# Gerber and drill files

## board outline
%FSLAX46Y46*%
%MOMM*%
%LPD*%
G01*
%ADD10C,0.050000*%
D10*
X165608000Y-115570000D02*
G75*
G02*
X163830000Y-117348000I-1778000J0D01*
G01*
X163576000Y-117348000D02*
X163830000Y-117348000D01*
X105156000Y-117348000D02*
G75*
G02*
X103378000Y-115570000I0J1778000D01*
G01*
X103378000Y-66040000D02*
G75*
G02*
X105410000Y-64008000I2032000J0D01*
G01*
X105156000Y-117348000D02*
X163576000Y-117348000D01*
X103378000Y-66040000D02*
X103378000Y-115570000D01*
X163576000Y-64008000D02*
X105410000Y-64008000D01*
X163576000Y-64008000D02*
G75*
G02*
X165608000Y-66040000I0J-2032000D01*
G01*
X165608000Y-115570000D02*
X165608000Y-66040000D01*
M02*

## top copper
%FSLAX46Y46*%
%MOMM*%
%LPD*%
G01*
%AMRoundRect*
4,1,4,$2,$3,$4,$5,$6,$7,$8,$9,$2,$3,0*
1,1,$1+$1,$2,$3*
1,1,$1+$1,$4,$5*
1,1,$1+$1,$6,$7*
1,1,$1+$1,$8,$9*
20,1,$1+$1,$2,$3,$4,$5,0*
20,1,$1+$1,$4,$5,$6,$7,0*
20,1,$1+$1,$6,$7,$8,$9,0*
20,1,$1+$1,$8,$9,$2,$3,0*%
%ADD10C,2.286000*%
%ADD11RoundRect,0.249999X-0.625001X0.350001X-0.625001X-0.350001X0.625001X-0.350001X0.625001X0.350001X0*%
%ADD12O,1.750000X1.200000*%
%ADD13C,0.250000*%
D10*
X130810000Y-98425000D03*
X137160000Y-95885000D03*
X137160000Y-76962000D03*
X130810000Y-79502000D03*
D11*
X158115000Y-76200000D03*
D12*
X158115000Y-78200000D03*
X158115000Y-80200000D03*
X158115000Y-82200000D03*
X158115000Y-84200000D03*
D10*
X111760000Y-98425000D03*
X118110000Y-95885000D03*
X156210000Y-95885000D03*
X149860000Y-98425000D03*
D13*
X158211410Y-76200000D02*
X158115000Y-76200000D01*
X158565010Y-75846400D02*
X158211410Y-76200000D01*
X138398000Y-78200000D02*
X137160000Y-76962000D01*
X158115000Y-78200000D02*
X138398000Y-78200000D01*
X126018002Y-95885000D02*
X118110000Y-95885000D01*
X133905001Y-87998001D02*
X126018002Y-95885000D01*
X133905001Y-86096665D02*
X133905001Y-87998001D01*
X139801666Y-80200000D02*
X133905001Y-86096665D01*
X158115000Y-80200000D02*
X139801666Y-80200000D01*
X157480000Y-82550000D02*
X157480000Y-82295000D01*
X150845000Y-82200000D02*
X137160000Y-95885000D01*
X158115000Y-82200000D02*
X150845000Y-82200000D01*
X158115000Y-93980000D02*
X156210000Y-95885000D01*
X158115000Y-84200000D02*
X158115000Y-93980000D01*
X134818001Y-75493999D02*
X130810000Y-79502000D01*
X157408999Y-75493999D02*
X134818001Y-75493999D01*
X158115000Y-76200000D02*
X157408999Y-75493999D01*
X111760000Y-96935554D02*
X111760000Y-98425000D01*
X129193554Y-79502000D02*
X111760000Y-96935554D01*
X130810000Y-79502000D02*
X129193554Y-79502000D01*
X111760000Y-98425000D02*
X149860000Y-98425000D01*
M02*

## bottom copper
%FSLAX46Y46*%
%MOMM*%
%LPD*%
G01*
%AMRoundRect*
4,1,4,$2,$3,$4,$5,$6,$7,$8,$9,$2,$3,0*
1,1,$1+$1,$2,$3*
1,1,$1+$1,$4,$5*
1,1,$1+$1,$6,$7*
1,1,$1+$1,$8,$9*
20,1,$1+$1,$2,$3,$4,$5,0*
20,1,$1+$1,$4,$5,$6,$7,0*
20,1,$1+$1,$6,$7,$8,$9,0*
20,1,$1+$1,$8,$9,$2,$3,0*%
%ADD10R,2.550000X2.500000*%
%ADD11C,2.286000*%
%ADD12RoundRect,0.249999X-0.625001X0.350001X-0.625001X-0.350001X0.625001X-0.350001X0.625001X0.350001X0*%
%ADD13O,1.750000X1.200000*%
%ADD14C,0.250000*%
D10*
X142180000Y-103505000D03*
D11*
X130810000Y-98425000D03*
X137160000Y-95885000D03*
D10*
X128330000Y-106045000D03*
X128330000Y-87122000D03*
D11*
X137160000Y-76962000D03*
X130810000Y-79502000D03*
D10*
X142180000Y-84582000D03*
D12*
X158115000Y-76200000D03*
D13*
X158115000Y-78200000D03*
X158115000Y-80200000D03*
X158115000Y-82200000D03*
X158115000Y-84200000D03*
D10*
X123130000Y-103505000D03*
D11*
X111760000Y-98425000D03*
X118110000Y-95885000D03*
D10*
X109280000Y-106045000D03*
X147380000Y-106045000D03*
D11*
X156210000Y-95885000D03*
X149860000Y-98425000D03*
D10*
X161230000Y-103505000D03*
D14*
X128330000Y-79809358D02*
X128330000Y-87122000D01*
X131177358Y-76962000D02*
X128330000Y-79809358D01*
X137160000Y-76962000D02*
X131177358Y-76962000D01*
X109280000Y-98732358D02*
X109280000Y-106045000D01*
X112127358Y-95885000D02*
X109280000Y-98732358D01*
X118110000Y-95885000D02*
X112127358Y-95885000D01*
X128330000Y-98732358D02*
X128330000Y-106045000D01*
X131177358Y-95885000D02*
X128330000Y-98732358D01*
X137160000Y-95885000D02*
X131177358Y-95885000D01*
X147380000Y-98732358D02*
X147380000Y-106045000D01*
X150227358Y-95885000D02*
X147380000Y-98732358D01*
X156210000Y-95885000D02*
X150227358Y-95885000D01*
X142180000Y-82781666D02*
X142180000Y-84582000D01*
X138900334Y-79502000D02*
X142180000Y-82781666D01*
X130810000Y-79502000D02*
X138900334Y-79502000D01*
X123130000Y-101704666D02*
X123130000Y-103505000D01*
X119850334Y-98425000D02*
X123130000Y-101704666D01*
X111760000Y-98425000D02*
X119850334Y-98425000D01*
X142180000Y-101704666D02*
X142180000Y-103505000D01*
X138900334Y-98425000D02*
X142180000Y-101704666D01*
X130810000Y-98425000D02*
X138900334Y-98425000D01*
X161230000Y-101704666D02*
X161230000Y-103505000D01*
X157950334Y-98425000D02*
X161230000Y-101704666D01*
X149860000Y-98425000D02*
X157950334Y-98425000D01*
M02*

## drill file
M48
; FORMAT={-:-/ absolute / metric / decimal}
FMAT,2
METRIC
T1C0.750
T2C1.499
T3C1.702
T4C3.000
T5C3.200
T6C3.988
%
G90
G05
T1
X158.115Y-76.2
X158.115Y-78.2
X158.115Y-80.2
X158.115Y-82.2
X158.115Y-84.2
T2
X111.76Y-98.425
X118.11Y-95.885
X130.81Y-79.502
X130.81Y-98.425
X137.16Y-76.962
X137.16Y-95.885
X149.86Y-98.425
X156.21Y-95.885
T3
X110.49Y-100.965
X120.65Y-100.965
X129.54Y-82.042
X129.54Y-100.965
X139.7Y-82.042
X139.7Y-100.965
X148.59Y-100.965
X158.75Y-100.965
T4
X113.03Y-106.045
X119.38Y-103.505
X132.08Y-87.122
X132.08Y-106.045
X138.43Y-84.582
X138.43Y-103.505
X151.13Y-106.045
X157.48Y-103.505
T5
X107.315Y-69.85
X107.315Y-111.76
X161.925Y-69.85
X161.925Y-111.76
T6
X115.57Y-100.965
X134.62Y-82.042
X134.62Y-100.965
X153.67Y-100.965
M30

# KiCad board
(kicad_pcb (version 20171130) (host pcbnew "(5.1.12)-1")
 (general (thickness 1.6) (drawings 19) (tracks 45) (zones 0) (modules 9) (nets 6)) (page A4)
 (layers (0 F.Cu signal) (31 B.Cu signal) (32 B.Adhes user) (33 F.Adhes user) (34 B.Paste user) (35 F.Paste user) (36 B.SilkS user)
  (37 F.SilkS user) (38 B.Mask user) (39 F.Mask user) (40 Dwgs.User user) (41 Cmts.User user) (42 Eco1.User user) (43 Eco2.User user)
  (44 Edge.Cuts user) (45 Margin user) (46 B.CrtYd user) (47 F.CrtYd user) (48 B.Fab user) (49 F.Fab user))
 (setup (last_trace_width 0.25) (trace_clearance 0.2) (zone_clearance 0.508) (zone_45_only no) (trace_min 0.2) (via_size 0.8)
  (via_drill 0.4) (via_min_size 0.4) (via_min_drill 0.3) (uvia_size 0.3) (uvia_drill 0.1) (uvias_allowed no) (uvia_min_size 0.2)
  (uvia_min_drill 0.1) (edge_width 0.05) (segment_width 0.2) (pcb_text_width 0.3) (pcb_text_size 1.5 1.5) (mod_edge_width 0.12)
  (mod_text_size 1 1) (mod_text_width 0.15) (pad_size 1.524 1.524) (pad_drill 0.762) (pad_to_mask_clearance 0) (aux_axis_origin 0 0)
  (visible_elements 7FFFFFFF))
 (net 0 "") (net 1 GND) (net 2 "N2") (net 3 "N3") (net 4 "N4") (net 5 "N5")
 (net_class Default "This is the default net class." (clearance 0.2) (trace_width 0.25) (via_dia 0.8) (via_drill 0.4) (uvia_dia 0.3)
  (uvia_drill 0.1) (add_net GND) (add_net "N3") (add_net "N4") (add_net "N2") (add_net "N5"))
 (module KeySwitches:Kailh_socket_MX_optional (layer F.Cu) (at 134.62 100.965)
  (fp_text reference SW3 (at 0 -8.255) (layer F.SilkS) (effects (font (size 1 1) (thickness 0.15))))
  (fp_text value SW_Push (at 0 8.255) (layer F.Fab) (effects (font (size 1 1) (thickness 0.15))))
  (pad 2 smd rect (at 7.56 2.54) (size 2.55 2.5) (layers B.Cu B.Paste B.Mask) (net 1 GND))
  (pad "" np_thru_hole circle (at -5.08 0) (size 1.7018 1.7018) (drill 1.7018) (layers *.Cu *.Mask))
  (pad "" np_thru_hole circle (at 5.08 0) (size 1.7018 1.7018) (drill 1.7018) (layers *.Cu *.Mask))
  (pad 2 thru_hole circle (at -3.81 -2.54) (size 2.286 2.286) (drill 1.4986) (layers *.Cu *.Mask) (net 1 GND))
  (pad "" np_thru_hole circle (at 0 0) (size 3.9878 3.9878) (drill 3.9878) (layers *.Cu *.Mask))
  (pad 1 thru_hole circle (at 2.54 -5.08) (size 2.286 2.286) (drill 1.4986) (layers *.Cu *.Mask) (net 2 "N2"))
  (pad "" np_thru_hole circle (at 3.81 2.54) (size 3 3) (drill 3) (layers *.Cu *.Mask))
  (pad "" np_thru_hole circle (at -2.54 5.08) (size 3 3) (drill 3) (layers *.Cu *.Mask))
  (pad 1 smd rect (at -6.29 5.08) (size 2.55 2.5) (layers B.Cu B.Paste B.Mask) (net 2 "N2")))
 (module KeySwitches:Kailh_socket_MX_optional (layer F.Cu) (at 134.62 82.042)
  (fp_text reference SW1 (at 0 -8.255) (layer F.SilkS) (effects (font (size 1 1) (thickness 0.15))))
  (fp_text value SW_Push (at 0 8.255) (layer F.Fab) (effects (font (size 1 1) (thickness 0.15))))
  (pad 1 smd rect (at -6.29 5.08) (size 2.55 2.5) (layers B.Cu B.Paste B.Mask) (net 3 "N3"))
  (pad "" np_thru_hole circle (at -2.54 5.08) (size 3 3) (drill 3) (layers *.Cu *.Mask))
  (pad "" np_thru_hole circle (at 3.81 2.54) (size 3 3) (drill 3) (layers *.Cu *.Mask))
  (pad 1 thru_hole circle (at 2.54 -5.08) (size 2.286 2.286) (drill 1.4986) (layers *.Cu *.Mask) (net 3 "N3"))
  (pad "" np_thru_hole circle (at 0 0) (size 3.9878 3.9878) (drill 3.9878) (layers *.Cu *.Mask))
  (pad 2 thru_hole circle (at -3.81 -2.54) (size 2.286 2.286) (drill 1.4986) (layers *.Cu *.Mask) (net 1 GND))
  (pad "" np_thru_hole circle (at 5.08 0) (size 1.7018 1.7018) (drill 1.7018) (layers *.Cu *.Mask))
  (pad "" np_thru_hole circle (at -5.08 0) (size 1.7018 1.7018) (drill 1.7018) (layers *.Cu *.Mask))
  (pad 2 smd rect (at 7.56 2.54) (size 2.55 2.5) (layers B.Cu B.Paste B.Mask) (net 1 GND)))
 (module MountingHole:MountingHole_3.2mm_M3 (layer F.Cu) (at 107.315 69.85)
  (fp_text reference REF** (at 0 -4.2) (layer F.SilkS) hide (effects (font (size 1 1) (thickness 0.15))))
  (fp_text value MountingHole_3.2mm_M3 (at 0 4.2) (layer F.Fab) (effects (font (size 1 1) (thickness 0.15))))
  (pad 1 np_thru_hole circle (at 0 0) (size 3.2 3.2) (drill 3.2) (layers *.Cu *.Mask)))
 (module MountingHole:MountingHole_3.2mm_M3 (layer F.Cu) (at 161.925 111.76)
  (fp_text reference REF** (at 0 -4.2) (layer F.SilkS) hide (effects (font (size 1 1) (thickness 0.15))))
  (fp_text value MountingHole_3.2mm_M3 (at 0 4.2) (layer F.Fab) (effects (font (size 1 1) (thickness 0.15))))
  (pad 1 np_thru_hole circle (at 0 0) (size 3.2 3.2) (drill 3.2) (layers *.Cu *.Mask)))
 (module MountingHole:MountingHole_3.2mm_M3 (layer F.Cu) (at 161.925 69.85)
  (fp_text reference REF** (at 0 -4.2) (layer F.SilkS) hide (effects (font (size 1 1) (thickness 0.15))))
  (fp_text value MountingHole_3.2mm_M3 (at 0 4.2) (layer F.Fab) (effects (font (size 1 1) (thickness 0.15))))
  (pad 1 np_thru_hole circle (at 0 0) (size 3.2 3.2) (drill 3.2) (layers *.Cu *.Mask)))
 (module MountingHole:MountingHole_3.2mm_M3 (layer F.Cu) (at 107.315 111.76)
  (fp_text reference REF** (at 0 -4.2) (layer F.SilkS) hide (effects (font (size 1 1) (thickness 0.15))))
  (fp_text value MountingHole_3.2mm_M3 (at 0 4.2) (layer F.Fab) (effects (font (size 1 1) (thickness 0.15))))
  (pad 1 np_thru_hole circle (at 0 0) (size 3.2 3.2) (drill 3.2) (layers *.Cu *.Mask)))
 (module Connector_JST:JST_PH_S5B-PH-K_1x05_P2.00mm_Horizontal (layer B.Cu) (at 158.115 76.2 270)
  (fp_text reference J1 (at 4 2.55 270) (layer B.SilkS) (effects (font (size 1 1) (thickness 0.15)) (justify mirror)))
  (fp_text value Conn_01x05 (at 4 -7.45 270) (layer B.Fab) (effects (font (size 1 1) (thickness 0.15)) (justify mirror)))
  (pad 1 thru_hole roundrect (at 0 0 270) (size 1.2 1.75) (drill 0.75) (layers *.Cu *.Mask) (roundrect_rratio 0.2083325) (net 1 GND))
  (pad 2 thru_hole oval (at 2 0 270) (size 1.2 1.75) (drill 0.75) (layers *.Cu *.Mask) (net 3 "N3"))
  (pad 3 thru_hole oval (at 4 0 270) (size 1.2 1.75) (drill 0.75) (layers *.Cu *.Mask) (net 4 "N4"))
  (pad 4 thru_hole oval (at 6 0 270) (size 1.2 1.75) (drill 0.75) (layers *.Cu *.Mask) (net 2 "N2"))
  (pad 5 thru_hole oval (at 8 0 270) (size 1.2 1.75) (drill 0.75) (layers *.Cu *.Mask) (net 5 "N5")))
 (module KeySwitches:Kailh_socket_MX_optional (layer F.Cu) (at 115.57 100.965)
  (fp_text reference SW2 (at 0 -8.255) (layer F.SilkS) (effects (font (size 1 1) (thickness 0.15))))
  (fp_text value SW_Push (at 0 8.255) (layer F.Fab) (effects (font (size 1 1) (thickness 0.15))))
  (pad 2 smd rect (at 7.56 2.54) (size 2.55 2.5) (layers B.Cu B.Paste B.Mask) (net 1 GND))
  (pad "" np_thru_hole circle (at -5.08 0) (size 1.7018 1.7018) (drill 1.7018) (layers *.Cu *.Mask))
  (pad "" np_thru_hole circle (at 5.08 0) (size 1.7018 1.7018) (drill 1.7018) (layers *.Cu *.Mask))
  (pad 2 thru_hole circle (at -3.81 -2.54) (size 2.286 2.286) (drill 1.4986) (layers *.Cu *.Mask) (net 1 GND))
  (pad "" np_thru_hole circle (at 0 0) (size 3.9878 3.9878) (drill 3.9878) (layers *.Cu *.Mask))
  (pad 1 thru_hole circle (at 2.54 -5.08) (size 2.286 2.286) (drill 1.4986) (layers *.Cu *.Mask) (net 4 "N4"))
  (pad "" np_thru_hole circle (at 3.81 2.54) (size 3 3) (drill 3) (layers *.Cu *.Mask))
  (pad "" np_thru_hole circle (at -2.54 5.08) (size 3 3) (drill 3) (layers *.Cu *.Mask))
  (pad 1 smd rect (at -6.29 5.08) (size 2.55 2.5) (layers B.Cu B.Paste B.Mask) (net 4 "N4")))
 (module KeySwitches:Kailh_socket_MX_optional (layer F.Cu) (at 153.67 100.965)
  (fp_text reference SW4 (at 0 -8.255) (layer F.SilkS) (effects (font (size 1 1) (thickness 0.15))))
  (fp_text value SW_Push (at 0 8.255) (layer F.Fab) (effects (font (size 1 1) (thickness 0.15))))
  (pad 1 smd rect (at -6.29 5.08) (size 2.55 2.5) (layers B.Cu B.Paste B.Mask) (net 5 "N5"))
  (pad "" np_thru_hole circle (at -2.54 5.08) (size 3 3) (drill 3) (layers *.Cu *.Mask))
  (pad "" np_thru_hole circle (at 3.81 2.54) (size 3 3) (drill 3) (layers *.Cu *.Mask))
  (pad 1 thru_hole circle (at 2.54 -5.08) (size 2.286 2.286) (drill 1.4986) (layers *.Cu *.Mask) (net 5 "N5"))
  (pad "" np_thru_hole circle (at 0 0) (size 3.9878 3.9878) (drill 3.9878) (layers *.Cu *.Mask))
  (pad 2 thru_hole circle (at -3.81 -2.54) (size 2.286 2.286) (drill 1.4986) (layers *.Cu *.Mask) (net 1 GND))
  (pad "" np_thru_hole circle (at 5.08 0) (size 1.7018 1.7018) (drill 1.7018) (layers *.Cu *.Mask))
  (pad "" np_thru_hole circle (at -5.08 0) (size 1.7018 1.7018) (drill 1.7018) (layers *.Cu *.Mask))
  (pad 2 smd rect (at 7.56 2.54) (size 2.55 2.5) (layers B.Cu B.Paste B.Mask) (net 1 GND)))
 (gr_arc (start 163.83 115.57) (end 163.83 117.348) (angle -90) (layer Edge.Cuts) (width 0.05))
 (gr_line (start 163.576 117.348) (end 163.83 117.348) (layer Edge.Cuts) (width 0.05))
 (gr_arc (start 105.156 115.57) (end 103.378 115.57) (angle -90) (layer Edge.Cuts) (width 0.05))
 (gr_arc (start 105.41 66.04) (end 105.41 64.008) (angle -90) (layer Edge.Cuts) (width 0.05))
 (gr_line (start 105.156 117.348) (end 163.576 117.348) (layer Edge.Cuts) (width 0.05))
 (gr_line (start 103.378 66.04) (end 103.378 115.57) (layer Edge.Cuts) (width 0.05))
 (gr_line (start 163.576 64.008) (end 105.41 64.008) (layer Edge.Cuts) (width 0.05))
 (gr_arc (start 163.576 66.04) (end 165.608 66.04) (angle -90) (layer Edge.Cuts) (width 0.05))
 (gr_line (start 165.608 115.57) (end 165.608 66.04) (layer Edge.Cuts) (width 0.05))
 (segment (start 158.21141 76.2) (end 158.115 76.2) (width 0.25) (layer F.Cu) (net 1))
 (segment (start 158.56501 75.8464) (end 158.21141 76.2) (width 0.25) (layer F.Cu) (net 1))
 (segment (start 138.398 78.2) (end 137.16 76.962) (width 0.25) (layer F.Cu) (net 3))
 (segment (start 158.115 78.2) (end 138.398 78.2) (width 0.25) (layer F.Cu) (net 3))
 (segment (start 128.33 79.809358) (end 128.33 87.122) (width 0.25) (layer B.Cu) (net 3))
 (segment (start 131.177358 76.962) (end 128.33 79.809358) (width 0.25) (layer B.Cu) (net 3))
 (segment (start 137.16 76.962) (end 131.177358 76.962) (width 0.25) (layer B.Cu) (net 3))
 (segment (start 126.018002 95.885) (end 118.11 95.885) (width 0.25) (layer F.Cu) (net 4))
 (segment (start 133.905001 87.998001) (end 126.018002 95.885) (width 0.25) (layer F.Cu) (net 4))
 (segment (start 133.905001 86.096665) (end 133.905001 87.998001) (width 0.25) (layer F.Cu) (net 4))
 (segment (start 139.801666 80.2) (end 133.905001 86.096665) (width 0.25) (layer F.Cu) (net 4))
 (segment (start 158.115 80.2) (end 139.801666 80.2) (width 0.25) (layer F.Cu) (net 4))
 (segment (start 109.28 98.732358) (end 109.28 106.045) (width 0.25) (layer B.Cu) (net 4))
 (segment (start 112.127358 95.885) (end 109.28 98.732358) (width 0.25) (layer B.Cu) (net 4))
 (segment (start 118.11 95.885) (end 112.127358 95.885) (width 0.25) (layer B.Cu) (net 4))
 (segment (start 157.48 82.55) (end 157.48 82.295) (width 0.25) (layer F.Cu) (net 2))
 (segment (start 150.845 82.2) (end 137.16 95.885) (width 0.25) (layer F.Cu) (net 2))
 (segment (start 158.115 82.2) (end 150.845 82.2) (width 0.25) (layer F.Cu) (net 2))
 (segment (start 128.33 98.732358) (end 128.33 106.045) (width 0.25) (layer B.Cu) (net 2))
 (segment (start 131.177358 95.885) (end 128.33 98.732358) (width 0.25) (layer B.Cu) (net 2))
 (segment (start 137.16 95.885) (end 131.177358 95.885) (width 0.25) (layer B.Cu) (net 2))
 (segment (start 158.115 93.98) (end 156.21 95.885) (width 0.25) (layer F.Cu) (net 5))
 (segment (start 158.115 84.2) (end 158.115 93.98) (width 0.25) (layer F.Cu) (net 5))
 (segment (start 147.38 98.732358) (end 147.38 106.045) (width 0.25) (layer B.Cu) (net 5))
 (segment (start 150.227358 95.885) (end 147.38 98.732358) (width 0.25) (layer B.Cu) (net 5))
 (segment (start 156.21 95.885) (end 150.227358 95.885) (width 0.25) (layer B.Cu) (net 5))
 (segment (start 134.818001 75.493999) (end 130.81 79.502) (width 0.25) (layer F.Cu) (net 1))
 (segment (start 157.408999 75.493999) (end 134.818001 75.493999) (width 0.25) (layer F.Cu) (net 1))
 (segment (start 158.115 76.2) (end 157.408999 75.493999) (width 0.25) (layer F.Cu) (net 1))
 (segment (start 111.76 96.935554) (end 111.76 98.425) (width 0.25) (layer F.Cu) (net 1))
 (segment (start 129.193554 79.502) (end 111.76 96.935554) (width 0.25) (layer F.Cu) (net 1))
 (segment (start 130.81 79.502) (end 129.193554 79.502) (width 0.25) (layer F.Cu) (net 1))
 (segment (start 111.76 98.425) (end 149.86 98.425) (width 0.25) (layer F.Cu) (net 1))
 (segment (start 142.18 82.781666) (end 142.18 84.582) (width 0.25) (layer B.Cu) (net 1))
 (segment (start 138.900334 79.502) (end 142.18 82.781666) (width 0.25) (layer B.Cu) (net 1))
 (segment (start 130.81 79.502) (end 138.900334 79.502) (width 0.25) (layer B.Cu) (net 1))
 (segment (start 123.13 101.704666) (end 123.13 103.505) (width 0.25) (layer B.Cu) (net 1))
 (segment (start 119.850334 98.425) (end 123.13 101.704666) (width 0.25) (layer B.Cu) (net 1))
 (segment (start 111.76 98.425) (end 119.850334 98.425) (width 0.25) (layer B.Cu) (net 1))
 (segment (start 142.18 101.704666) (end 142.18 103.505) (width 0.25) (layer B.Cu) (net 1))
 (segment (start 138.900334 98.425) (end 142.18 101.704666) (width 0.25) (layer B.Cu) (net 1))
 (segment (start 130.81 98.425) (end 138.900334 98.425) (width 0.25) (layer B.Cu) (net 1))
 (segment (start 161.23 101.704666) (end 161.23 103.505) (width 0.25) (layer B.Cu) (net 1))
 (segment (start 157.950334 98.425) (end 161.23 101.704666) (width 0.25) (layer B.Cu) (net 1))
 (segment (start 149.86 98.425) (end 157.950334 98.425) (width 0.25) (layer B.Cu) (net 1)))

